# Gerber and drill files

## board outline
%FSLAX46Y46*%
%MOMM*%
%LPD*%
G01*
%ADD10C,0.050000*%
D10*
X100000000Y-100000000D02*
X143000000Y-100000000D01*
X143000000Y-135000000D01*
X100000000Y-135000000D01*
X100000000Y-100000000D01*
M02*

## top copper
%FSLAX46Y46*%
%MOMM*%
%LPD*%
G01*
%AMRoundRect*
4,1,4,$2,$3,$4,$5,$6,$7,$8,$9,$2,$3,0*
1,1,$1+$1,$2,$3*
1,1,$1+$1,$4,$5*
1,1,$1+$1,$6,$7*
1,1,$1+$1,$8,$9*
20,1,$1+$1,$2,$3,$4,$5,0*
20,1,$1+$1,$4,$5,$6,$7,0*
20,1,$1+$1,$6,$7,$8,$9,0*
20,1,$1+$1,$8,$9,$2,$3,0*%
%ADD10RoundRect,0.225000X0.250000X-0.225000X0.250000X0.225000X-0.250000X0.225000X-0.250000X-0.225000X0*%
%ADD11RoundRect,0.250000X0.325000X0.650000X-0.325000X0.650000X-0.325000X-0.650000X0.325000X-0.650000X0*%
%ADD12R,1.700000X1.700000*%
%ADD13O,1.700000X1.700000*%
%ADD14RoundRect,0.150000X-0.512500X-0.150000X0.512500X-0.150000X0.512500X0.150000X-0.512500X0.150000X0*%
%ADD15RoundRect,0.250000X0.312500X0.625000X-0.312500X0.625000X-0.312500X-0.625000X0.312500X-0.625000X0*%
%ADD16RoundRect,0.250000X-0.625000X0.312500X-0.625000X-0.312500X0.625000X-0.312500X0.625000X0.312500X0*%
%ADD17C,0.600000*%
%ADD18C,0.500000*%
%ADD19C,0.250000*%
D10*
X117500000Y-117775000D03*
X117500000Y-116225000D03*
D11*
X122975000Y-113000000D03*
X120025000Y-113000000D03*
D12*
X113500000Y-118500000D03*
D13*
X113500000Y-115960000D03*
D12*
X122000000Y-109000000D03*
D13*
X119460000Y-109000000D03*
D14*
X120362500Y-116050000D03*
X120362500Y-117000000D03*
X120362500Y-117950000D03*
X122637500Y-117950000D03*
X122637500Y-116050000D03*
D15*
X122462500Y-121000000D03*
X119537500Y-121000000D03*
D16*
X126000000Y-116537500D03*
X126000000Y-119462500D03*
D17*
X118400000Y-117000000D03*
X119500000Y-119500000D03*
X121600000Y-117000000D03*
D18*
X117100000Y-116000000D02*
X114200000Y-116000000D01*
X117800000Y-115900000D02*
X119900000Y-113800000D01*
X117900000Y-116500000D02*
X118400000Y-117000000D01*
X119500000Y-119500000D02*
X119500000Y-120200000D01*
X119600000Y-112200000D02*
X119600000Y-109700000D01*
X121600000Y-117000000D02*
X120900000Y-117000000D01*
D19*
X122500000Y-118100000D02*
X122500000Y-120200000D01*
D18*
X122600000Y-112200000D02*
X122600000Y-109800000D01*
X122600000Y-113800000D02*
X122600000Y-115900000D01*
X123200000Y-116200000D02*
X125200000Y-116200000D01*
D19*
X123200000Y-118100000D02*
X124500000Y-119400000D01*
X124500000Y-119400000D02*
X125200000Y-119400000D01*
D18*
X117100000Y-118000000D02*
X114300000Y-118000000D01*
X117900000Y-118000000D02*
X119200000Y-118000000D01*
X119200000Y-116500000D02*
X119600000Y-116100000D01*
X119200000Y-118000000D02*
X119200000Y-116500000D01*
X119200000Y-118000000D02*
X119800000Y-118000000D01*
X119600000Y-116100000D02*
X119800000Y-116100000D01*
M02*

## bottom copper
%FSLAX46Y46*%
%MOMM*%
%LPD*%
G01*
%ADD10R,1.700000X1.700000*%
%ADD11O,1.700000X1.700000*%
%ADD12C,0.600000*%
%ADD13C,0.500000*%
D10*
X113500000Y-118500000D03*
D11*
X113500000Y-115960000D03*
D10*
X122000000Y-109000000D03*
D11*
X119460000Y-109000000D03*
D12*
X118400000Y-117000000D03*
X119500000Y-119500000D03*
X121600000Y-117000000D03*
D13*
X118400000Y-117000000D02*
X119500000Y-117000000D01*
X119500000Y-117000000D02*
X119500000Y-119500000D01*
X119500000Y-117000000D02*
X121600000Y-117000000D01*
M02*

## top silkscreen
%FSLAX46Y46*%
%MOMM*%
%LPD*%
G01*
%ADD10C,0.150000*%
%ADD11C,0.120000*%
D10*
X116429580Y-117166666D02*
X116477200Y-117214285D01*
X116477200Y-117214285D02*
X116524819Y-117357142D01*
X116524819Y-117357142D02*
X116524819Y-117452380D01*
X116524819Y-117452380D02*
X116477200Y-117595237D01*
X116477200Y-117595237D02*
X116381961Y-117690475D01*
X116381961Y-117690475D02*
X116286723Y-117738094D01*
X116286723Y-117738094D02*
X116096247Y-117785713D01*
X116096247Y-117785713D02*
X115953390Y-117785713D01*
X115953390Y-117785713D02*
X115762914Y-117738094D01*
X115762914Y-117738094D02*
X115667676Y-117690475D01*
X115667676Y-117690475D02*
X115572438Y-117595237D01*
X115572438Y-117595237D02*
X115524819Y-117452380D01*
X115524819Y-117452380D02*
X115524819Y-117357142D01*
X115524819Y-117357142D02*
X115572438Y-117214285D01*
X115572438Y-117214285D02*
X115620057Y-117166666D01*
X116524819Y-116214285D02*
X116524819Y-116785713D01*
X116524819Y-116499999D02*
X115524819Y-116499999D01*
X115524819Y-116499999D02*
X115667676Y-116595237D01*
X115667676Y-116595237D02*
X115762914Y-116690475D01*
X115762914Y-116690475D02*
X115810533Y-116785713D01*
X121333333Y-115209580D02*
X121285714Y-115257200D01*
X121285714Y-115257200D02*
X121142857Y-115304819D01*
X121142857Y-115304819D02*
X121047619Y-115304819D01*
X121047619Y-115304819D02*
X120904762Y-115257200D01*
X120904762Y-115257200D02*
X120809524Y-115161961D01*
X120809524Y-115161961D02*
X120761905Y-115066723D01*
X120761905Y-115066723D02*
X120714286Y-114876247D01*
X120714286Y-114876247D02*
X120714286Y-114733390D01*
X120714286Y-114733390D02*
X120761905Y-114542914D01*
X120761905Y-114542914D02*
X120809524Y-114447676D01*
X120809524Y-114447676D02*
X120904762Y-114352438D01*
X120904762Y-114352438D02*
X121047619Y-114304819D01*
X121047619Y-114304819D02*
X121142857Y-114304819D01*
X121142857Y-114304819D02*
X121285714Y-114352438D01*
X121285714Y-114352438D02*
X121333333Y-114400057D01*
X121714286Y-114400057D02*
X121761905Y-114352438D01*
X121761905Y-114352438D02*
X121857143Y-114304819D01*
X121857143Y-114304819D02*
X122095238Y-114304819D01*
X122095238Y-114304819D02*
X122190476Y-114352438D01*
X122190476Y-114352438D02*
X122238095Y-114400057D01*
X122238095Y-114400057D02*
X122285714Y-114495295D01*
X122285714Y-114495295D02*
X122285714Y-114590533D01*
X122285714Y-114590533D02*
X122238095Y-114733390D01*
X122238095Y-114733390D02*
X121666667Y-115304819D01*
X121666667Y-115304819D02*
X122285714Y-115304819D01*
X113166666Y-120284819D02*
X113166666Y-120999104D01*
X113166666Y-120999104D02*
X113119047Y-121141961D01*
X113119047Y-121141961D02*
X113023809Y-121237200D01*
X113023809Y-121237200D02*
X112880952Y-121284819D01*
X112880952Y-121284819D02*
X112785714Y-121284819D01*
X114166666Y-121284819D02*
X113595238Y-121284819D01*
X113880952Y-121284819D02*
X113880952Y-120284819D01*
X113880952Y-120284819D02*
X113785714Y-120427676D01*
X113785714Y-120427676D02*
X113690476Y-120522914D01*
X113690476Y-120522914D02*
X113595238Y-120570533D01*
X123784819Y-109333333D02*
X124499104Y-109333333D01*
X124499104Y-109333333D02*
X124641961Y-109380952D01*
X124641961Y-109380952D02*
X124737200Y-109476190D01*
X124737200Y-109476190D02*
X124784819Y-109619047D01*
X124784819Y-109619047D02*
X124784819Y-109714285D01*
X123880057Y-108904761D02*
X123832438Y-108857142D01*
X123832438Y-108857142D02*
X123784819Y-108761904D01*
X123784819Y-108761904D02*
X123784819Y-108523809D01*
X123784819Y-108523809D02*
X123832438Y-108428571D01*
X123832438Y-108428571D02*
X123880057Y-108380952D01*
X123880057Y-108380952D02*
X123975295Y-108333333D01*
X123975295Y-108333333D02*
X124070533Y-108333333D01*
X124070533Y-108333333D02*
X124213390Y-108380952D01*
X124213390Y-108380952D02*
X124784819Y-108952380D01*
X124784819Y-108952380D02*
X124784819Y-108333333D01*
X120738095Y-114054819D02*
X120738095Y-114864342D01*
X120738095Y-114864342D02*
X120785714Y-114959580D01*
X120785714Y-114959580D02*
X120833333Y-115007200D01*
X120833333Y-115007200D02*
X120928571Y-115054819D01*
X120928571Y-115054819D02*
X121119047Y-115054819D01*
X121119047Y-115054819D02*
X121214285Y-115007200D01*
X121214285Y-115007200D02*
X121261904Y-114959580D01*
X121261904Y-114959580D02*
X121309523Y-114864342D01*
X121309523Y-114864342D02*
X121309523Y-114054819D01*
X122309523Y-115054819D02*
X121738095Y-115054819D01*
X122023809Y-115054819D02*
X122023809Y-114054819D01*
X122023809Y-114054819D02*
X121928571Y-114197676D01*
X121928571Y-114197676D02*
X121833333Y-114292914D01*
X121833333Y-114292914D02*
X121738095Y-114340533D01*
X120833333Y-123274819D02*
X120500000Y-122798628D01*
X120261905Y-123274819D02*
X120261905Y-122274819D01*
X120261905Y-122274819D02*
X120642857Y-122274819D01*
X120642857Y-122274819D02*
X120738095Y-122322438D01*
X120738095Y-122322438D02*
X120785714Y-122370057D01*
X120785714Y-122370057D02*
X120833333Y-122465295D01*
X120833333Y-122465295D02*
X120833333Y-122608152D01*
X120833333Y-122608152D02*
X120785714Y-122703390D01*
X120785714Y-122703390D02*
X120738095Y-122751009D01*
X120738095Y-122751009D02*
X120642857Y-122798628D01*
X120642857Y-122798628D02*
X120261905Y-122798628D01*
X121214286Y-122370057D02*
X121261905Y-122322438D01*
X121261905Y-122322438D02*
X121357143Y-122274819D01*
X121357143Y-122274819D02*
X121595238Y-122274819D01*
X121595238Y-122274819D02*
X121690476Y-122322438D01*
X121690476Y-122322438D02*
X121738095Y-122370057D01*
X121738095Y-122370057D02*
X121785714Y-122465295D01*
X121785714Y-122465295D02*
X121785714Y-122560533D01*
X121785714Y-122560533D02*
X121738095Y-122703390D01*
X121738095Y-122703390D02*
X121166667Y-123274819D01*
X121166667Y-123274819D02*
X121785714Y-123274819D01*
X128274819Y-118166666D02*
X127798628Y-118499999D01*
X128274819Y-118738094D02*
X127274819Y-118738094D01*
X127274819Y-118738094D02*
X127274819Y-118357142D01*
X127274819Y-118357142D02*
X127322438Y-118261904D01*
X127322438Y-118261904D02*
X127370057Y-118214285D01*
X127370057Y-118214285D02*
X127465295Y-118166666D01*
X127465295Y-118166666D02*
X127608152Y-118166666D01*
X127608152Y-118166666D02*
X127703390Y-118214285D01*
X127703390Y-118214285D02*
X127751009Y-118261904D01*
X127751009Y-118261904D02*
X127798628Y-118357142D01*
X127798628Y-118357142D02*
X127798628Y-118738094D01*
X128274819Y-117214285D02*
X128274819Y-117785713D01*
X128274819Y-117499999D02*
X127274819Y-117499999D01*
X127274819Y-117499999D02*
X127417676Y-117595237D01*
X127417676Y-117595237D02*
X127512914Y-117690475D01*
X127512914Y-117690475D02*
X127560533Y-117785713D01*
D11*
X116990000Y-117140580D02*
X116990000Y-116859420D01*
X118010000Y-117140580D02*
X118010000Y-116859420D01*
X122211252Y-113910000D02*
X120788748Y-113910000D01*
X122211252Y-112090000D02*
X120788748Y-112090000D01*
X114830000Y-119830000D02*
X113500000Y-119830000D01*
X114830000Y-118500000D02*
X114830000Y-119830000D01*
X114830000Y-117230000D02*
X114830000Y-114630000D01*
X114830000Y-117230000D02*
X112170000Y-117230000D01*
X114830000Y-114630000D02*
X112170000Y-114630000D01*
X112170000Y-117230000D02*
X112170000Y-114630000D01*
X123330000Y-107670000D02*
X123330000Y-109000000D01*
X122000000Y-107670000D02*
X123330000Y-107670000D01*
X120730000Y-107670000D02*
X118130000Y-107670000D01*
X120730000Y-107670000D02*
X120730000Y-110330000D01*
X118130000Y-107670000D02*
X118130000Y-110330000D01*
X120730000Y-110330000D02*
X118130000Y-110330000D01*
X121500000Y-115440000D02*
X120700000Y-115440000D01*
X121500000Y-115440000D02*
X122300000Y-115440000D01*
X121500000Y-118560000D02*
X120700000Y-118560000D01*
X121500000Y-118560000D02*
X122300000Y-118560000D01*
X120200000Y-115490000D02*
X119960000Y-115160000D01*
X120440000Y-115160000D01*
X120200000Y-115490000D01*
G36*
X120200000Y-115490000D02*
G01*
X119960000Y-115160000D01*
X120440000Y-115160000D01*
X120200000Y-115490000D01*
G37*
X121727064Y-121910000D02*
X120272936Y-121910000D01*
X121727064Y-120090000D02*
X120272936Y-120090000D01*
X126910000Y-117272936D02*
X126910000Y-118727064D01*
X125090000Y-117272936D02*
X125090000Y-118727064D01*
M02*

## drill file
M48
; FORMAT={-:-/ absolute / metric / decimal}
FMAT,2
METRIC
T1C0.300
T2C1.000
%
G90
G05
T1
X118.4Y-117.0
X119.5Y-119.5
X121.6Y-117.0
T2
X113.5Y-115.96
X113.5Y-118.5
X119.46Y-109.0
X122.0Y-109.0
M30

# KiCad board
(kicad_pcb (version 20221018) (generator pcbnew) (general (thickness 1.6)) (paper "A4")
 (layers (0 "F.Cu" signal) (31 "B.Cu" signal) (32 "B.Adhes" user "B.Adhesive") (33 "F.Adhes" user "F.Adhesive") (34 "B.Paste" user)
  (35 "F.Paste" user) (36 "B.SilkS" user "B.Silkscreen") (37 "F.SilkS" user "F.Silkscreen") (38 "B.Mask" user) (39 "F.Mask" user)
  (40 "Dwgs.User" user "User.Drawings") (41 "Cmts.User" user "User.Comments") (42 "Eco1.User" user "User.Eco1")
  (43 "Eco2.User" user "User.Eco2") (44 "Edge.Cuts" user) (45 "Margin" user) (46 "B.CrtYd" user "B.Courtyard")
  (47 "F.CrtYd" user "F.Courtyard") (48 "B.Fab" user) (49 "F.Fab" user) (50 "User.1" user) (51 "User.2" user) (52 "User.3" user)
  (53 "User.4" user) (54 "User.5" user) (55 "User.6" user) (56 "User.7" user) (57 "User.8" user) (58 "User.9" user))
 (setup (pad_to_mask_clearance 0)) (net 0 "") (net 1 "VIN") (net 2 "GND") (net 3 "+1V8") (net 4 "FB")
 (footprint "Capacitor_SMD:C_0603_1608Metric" (layer "F.Cu") (at 117.5 117 90)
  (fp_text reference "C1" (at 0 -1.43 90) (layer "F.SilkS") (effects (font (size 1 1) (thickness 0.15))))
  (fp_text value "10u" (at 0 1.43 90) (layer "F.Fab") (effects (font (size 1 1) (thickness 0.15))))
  (fp_line (start -0.14058 -0.51) (end 0.14058 -0.51) (stroke (width 0.12) (type solid)) (layer "F.SilkS"))
  (fp_line (start -0.14058 0.51) (end 0.14058 0.51) (stroke (width 0.12) (type solid)) (layer "F.SilkS"))
  (pad "1" smd roundrect (at -0.775 0 90) (size 0.9 0.95) (layers "F.Cu" "F.Paste" "F.Mask") (roundrect_rratio 0.25) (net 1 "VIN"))
  (pad "2" smd roundrect (at 0.775 0 90) (size 0.9 0.95) (layers "F.Cu" "F.Paste" "F.Mask") (roundrect_rratio 0.25) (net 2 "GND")))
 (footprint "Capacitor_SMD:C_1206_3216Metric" (layer "F.Cu") (at 121.5 113 180)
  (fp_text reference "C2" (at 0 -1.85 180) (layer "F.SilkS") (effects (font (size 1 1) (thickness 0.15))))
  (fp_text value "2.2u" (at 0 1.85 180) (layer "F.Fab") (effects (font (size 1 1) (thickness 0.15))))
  (fp_line (start -0.711252 -0.91) (end 0.711252 -0.91) (stroke (width 0.12) (type solid)) (layer "F.SilkS"))
  (fp_line (start -0.711252 0.91) (end 0.711252 0.91) (stroke (width 0.12) (type solid)) (layer "F.SilkS"))
  (pad "1" smd roundrect (at -1.475 0 180) (size 1.15 1.8) (layers "F.Cu" "F.Paste" "F.Mask") (roundrect_rratio 0.217391) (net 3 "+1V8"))
  (pad "2" smd roundrect (at 1.475 0 180) (size 1.15 1.8) (layers "F.Cu" "F.Paste" "F.Mask") (roundrect_rratio 0.217391) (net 2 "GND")))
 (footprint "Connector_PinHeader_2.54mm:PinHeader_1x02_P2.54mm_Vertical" (layer "F.Cu") (at 113.5 118.5 180)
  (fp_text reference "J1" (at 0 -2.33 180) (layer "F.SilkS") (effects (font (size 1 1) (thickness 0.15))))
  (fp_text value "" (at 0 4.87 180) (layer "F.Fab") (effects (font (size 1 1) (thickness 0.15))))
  (fp_line (start -1.33 -1.33) (end 0 -1.33) (stroke (width 0.12) (type solid)) (layer "F.SilkS"))
  (fp_line (start -1.33 0) (end -1.33 -1.33) (stroke (width 0.12) (type solid)) (layer "F.SilkS"))
  (fp_line (start -1.33 1.27) (end -1.33 3.87) (stroke (width 0.12) (type solid)) (layer "F.SilkS"))
  (fp_line (start -1.33 1.27) (end 1.33 1.27) (stroke (width 0.12) (type solid)) (layer "F.SilkS"))
  (fp_line (start -1.33 3.87) (end 1.33 3.87) (stroke (width 0.12) (type solid)) (layer "F.SilkS"))
  (fp_line (start 1.33 1.27) (end 1.33 3.87) (stroke (width 0.12) (type solid)) (layer "F.SilkS"))
  (pad "1" thru_hole rect (at 0 0 180) (size 1.7 1.7) (drill 1) (layers "*.Cu" "*.Mask") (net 1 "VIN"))
  (pad "2" thru_hole oval (at 0 2.54 180) (size 1.7 1.7) (drill 1) (layers "*.Cu" "*.Mask") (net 2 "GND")))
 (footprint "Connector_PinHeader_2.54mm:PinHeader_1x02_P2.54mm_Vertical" (layer "F.Cu") (at 122 109 -90)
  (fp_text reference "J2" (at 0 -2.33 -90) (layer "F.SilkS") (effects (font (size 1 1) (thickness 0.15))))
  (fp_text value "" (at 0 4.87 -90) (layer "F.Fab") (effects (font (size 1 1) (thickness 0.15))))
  (fp_line (start -1.33 -1.33) (end 0 -1.33) (stroke (width 0.12) (type solid)) (layer "F.SilkS"))
  (fp_line (start -1.33 0) (end -1.33 -1.33) (stroke (width 0.12) (type solid)) (layer "F.SilkS"))
  (fp_line (start -1.33 1.27) (end -1.33 3.87) (stroke (width 0.12) (type solid)) (layer "F.SilkS"))
  (fp_line (start -1.33 1.27) (end 1.33 1.27) (stroke (width 0.12) (type solid)) (layer "F.SilkS"))
  (fp_line (start -1.33 3.87) (end 1.33 3.87) (stroke (width 0.12) (type solid)) (layer "F.SilkS"))
  (fp_line (start 1.33 1.27) (end 1.33 3.87) (stroke (width 0.12) (type solid)) (layer "F.SilkS"))
  (pad "1" thru_hole rect (at 0 0 270) (size 1.7 1.7) (drill 1) (layers "*.Cu" "*.Mask") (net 3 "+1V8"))
  (pad "2" thru_hole oval (at 0 2.54 270) (size 1.7 1.7) (drill 1) (layers "*.Cu" "*.Mask") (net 2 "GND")))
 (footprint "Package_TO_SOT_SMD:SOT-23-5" (layer "F.Cu") (at 121.5 117)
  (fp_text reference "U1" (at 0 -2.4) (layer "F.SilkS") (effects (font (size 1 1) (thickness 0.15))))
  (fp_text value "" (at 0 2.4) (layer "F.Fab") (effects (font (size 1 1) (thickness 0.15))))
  (fp_line (start 0 -1.56) (end -0.8 -1.56) (stroke (width 0.12) (type solid)) (layer "F.SilkS"))
  (fp_line (start 0 -1.56) (end 0.8 -1.56) (stroke (width 0.12) (type solid)) (layer "F.SilkS"))
  (fp_line (start 0 1.56) (end -0.8 1.56) (stroke (width 0.12) (type solid)) (layer "F.SilkS"))
  (fp_line (start 0 1.56) (end 0.8 1.56) (stroke (width 0.12) (type solid)) (layer "F.SilkS"))
  (fp_poly
   (pts (xy -1.3 -1.51) (xy -1.54 -1.84) (xy -1.06 -1.84) (xy -1.3 -1.51)) (stroke (width 0.12) (type solid)) (fill solid) (layer "F.SilkS"))
  (pad "1" smd roundrect (at -1.1375 -0.95) (size 1.325 0.6) (layers "F.Cu" "F.Paste" "F.Mask") (roundrect_rratio 0.25) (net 1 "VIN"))
  (pad "2" smd roundrect (at -1.1375 0) (size 1.325 0.6) (layers "F.Cu" "F.Paste" "F.Mask") (roundrect_rratio 0.25) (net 2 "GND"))
  (pad "3" smd roundrect (at -1.1375 0.95) (size 1.325 0.6) (layers "F.Cu" "F.Paste" "F.Mask") (roundrect_rratio 0.25) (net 1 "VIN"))
  (pad "4" smd roundrect (at 1.1375 0.95) (size 1.325 0.6) (layers "F.Cu" "F.Paste" "F.Mask") (roundrect_rratio 0.25) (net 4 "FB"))
  (pad "5" smd roundrect (at 1.1375 -0.95) (size 1.325 0.6) (layers "F.Cu" "F.Paste" "F.Mask") (roundrect_rratio 0.25) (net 3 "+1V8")))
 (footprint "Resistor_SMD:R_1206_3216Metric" (layer "F.Cu") (at 121 121 180)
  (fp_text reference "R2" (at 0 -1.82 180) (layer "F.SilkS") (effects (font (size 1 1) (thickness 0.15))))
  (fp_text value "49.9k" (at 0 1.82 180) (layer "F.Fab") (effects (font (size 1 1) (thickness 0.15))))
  (fp_line (start -0.727064 -0.91) (end 0.727064 -0.91) (stroke (width 0.12) (type solid)) (layer "F.SilkS"))
  (fp_line (start -0.727064 0.91) (end 0.727064 0.91) (stroke (width 0.12) (type solid)) (layer "F.SilkS"))
  (pad "1" smd roundrect (at -1.4625 0 180) (size 1.125 1.75) (layers "F.Cu" "F.Paste" "F.Mask") (roundrect_rratio 0.222222) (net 4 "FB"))
  (pad "2" smd roundrect (at 1.4625 0 180) (size 1.125 1.75) (layers "F.Cu" "F.Paste" "F.Mask") (roundrect_rratio 0.222222) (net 2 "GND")))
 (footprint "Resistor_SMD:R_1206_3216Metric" (layer "F.Cu") (at 126 118 -90)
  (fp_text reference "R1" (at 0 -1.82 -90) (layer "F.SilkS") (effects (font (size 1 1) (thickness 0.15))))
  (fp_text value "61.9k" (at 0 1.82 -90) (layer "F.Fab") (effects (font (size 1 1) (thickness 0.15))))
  (fp_line (start -0.727064 -0.91) (end 0.727064 -0.91) (stroke (width 0.12) (type solid)) (layer "F.SilkS"))
  (fp_line (start -0.727064 0.91) (end 0.727064 0.91) (stroke (width 0.12) (type solid)) (layer "F.SilkS"))
  (pad "1" smd roundrect (at -1.4625 0 270) (size 1.125 1.75) (layers "F.Cu" "F.Paste" "F.Mask") (roundrect_rratio 0.222222) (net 3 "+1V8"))
  (pad "2" smd roundrect (at 1.4625 0 270) (size 1.125 1.75) (layers "F.Cu" "F.Paste" "F.Mask") (roundrect_rratio 0.222222) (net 4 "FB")))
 (gr_rect (start 100 100) (end 143 135) (stroke (width 0.05) (type default)) (fill none) (layer "Edge.Cuts"))
 (segment (start 117.1 116) (end 114.2 116) (width 0.5) (layer "F.Cu") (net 2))
 (segment (start 117.8 115.9) (end 119.9 113.8) (width 0.5) (layer "F.Cu") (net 2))
 (segment (start 117.9 116.5) (end 118.4 117) (width 0.5) (layer "F.Cu") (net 2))
 (segment (start 119.5 119.5) (end 119.5 120.2) (width 0.5) (layer "F.Cu") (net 2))
 (segment (start 119.6 112.2) (end 119.6 109.7) (width 0.5) (layer "F.Cu") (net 2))
 (segment (start 121.6 117) (end 120.9 117) (width 0.5) (layer "F.Cu") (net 2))
 (segment (start 122.5 118.1) (end 122.5 120.2) (width 0.25) (layer "F.Cu") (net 4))
 (segment (start 122.6 112.2) (end 122.6 109.8) (width 0.5) (layer "F.Cu") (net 3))
 (segment (start 122.6 113.8) (end 122.6 115.9) (width 0.5) (layer "F.Cu") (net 3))
 (segment (start 123.2 116.2) (end 125.2 116.2) (width 0.5) (layer "F.Cu") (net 3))
 (segment (start 123.2 118.1) (end 124.5 119.4) (width 0.25) (layer "F.Cu") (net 4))
 (segment (start 124.5 119.4) (end 125.2 119.4) (width 0.25) (layer "F.Cu") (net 4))
 (via (at 118.4 117) (size 0.6) (drill 0.3) (layers "F.Cu" "B.Cu") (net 2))
 (via (at 119.5 119.5) (size 0.6) (drill 0.3) (layers "F.Cu" "B.Cu") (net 2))
 (via (at 121.6 117) (size 0.6) (drill 0.3) (layers "F.Cu" "B.Cu") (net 2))
 (segment (start 117.1 118) (end 114.3 118) (width 0.5) (layer "F.Cu") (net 1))
 (segment (start 117.9 118) (end 119.2 118) (width 0.5) (layer "F.Cu") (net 1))
 (segment (start 118.4 117) (end 119.5 117) (width 0.5) (layer "B.Cu") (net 2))
 (segment (start 119.2 116.5) (end 119.6 116.1) (width 0.5) (layer "F.Cu") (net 1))
 (segment (start 119.2 118) (end 119.2 116.5) (width 0.5) (layer "F.Cu") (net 1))
 (segment (start 119.2 118) (end 119.8 118) (width 0.5) (layer "F.Cu") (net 1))
 (segment (start 119.5 117) (end 119.5 119.5) (width 0.5) (layer "B.Cu") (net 2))
 (segment (start 119.5 117) (end 121.6 117) (width 0.5) (layer "B.Cu") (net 2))
 (segment (start 119.6 116.1) (end 119.8 116.1) (width 0.5) (layer "F.Cu") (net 1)))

